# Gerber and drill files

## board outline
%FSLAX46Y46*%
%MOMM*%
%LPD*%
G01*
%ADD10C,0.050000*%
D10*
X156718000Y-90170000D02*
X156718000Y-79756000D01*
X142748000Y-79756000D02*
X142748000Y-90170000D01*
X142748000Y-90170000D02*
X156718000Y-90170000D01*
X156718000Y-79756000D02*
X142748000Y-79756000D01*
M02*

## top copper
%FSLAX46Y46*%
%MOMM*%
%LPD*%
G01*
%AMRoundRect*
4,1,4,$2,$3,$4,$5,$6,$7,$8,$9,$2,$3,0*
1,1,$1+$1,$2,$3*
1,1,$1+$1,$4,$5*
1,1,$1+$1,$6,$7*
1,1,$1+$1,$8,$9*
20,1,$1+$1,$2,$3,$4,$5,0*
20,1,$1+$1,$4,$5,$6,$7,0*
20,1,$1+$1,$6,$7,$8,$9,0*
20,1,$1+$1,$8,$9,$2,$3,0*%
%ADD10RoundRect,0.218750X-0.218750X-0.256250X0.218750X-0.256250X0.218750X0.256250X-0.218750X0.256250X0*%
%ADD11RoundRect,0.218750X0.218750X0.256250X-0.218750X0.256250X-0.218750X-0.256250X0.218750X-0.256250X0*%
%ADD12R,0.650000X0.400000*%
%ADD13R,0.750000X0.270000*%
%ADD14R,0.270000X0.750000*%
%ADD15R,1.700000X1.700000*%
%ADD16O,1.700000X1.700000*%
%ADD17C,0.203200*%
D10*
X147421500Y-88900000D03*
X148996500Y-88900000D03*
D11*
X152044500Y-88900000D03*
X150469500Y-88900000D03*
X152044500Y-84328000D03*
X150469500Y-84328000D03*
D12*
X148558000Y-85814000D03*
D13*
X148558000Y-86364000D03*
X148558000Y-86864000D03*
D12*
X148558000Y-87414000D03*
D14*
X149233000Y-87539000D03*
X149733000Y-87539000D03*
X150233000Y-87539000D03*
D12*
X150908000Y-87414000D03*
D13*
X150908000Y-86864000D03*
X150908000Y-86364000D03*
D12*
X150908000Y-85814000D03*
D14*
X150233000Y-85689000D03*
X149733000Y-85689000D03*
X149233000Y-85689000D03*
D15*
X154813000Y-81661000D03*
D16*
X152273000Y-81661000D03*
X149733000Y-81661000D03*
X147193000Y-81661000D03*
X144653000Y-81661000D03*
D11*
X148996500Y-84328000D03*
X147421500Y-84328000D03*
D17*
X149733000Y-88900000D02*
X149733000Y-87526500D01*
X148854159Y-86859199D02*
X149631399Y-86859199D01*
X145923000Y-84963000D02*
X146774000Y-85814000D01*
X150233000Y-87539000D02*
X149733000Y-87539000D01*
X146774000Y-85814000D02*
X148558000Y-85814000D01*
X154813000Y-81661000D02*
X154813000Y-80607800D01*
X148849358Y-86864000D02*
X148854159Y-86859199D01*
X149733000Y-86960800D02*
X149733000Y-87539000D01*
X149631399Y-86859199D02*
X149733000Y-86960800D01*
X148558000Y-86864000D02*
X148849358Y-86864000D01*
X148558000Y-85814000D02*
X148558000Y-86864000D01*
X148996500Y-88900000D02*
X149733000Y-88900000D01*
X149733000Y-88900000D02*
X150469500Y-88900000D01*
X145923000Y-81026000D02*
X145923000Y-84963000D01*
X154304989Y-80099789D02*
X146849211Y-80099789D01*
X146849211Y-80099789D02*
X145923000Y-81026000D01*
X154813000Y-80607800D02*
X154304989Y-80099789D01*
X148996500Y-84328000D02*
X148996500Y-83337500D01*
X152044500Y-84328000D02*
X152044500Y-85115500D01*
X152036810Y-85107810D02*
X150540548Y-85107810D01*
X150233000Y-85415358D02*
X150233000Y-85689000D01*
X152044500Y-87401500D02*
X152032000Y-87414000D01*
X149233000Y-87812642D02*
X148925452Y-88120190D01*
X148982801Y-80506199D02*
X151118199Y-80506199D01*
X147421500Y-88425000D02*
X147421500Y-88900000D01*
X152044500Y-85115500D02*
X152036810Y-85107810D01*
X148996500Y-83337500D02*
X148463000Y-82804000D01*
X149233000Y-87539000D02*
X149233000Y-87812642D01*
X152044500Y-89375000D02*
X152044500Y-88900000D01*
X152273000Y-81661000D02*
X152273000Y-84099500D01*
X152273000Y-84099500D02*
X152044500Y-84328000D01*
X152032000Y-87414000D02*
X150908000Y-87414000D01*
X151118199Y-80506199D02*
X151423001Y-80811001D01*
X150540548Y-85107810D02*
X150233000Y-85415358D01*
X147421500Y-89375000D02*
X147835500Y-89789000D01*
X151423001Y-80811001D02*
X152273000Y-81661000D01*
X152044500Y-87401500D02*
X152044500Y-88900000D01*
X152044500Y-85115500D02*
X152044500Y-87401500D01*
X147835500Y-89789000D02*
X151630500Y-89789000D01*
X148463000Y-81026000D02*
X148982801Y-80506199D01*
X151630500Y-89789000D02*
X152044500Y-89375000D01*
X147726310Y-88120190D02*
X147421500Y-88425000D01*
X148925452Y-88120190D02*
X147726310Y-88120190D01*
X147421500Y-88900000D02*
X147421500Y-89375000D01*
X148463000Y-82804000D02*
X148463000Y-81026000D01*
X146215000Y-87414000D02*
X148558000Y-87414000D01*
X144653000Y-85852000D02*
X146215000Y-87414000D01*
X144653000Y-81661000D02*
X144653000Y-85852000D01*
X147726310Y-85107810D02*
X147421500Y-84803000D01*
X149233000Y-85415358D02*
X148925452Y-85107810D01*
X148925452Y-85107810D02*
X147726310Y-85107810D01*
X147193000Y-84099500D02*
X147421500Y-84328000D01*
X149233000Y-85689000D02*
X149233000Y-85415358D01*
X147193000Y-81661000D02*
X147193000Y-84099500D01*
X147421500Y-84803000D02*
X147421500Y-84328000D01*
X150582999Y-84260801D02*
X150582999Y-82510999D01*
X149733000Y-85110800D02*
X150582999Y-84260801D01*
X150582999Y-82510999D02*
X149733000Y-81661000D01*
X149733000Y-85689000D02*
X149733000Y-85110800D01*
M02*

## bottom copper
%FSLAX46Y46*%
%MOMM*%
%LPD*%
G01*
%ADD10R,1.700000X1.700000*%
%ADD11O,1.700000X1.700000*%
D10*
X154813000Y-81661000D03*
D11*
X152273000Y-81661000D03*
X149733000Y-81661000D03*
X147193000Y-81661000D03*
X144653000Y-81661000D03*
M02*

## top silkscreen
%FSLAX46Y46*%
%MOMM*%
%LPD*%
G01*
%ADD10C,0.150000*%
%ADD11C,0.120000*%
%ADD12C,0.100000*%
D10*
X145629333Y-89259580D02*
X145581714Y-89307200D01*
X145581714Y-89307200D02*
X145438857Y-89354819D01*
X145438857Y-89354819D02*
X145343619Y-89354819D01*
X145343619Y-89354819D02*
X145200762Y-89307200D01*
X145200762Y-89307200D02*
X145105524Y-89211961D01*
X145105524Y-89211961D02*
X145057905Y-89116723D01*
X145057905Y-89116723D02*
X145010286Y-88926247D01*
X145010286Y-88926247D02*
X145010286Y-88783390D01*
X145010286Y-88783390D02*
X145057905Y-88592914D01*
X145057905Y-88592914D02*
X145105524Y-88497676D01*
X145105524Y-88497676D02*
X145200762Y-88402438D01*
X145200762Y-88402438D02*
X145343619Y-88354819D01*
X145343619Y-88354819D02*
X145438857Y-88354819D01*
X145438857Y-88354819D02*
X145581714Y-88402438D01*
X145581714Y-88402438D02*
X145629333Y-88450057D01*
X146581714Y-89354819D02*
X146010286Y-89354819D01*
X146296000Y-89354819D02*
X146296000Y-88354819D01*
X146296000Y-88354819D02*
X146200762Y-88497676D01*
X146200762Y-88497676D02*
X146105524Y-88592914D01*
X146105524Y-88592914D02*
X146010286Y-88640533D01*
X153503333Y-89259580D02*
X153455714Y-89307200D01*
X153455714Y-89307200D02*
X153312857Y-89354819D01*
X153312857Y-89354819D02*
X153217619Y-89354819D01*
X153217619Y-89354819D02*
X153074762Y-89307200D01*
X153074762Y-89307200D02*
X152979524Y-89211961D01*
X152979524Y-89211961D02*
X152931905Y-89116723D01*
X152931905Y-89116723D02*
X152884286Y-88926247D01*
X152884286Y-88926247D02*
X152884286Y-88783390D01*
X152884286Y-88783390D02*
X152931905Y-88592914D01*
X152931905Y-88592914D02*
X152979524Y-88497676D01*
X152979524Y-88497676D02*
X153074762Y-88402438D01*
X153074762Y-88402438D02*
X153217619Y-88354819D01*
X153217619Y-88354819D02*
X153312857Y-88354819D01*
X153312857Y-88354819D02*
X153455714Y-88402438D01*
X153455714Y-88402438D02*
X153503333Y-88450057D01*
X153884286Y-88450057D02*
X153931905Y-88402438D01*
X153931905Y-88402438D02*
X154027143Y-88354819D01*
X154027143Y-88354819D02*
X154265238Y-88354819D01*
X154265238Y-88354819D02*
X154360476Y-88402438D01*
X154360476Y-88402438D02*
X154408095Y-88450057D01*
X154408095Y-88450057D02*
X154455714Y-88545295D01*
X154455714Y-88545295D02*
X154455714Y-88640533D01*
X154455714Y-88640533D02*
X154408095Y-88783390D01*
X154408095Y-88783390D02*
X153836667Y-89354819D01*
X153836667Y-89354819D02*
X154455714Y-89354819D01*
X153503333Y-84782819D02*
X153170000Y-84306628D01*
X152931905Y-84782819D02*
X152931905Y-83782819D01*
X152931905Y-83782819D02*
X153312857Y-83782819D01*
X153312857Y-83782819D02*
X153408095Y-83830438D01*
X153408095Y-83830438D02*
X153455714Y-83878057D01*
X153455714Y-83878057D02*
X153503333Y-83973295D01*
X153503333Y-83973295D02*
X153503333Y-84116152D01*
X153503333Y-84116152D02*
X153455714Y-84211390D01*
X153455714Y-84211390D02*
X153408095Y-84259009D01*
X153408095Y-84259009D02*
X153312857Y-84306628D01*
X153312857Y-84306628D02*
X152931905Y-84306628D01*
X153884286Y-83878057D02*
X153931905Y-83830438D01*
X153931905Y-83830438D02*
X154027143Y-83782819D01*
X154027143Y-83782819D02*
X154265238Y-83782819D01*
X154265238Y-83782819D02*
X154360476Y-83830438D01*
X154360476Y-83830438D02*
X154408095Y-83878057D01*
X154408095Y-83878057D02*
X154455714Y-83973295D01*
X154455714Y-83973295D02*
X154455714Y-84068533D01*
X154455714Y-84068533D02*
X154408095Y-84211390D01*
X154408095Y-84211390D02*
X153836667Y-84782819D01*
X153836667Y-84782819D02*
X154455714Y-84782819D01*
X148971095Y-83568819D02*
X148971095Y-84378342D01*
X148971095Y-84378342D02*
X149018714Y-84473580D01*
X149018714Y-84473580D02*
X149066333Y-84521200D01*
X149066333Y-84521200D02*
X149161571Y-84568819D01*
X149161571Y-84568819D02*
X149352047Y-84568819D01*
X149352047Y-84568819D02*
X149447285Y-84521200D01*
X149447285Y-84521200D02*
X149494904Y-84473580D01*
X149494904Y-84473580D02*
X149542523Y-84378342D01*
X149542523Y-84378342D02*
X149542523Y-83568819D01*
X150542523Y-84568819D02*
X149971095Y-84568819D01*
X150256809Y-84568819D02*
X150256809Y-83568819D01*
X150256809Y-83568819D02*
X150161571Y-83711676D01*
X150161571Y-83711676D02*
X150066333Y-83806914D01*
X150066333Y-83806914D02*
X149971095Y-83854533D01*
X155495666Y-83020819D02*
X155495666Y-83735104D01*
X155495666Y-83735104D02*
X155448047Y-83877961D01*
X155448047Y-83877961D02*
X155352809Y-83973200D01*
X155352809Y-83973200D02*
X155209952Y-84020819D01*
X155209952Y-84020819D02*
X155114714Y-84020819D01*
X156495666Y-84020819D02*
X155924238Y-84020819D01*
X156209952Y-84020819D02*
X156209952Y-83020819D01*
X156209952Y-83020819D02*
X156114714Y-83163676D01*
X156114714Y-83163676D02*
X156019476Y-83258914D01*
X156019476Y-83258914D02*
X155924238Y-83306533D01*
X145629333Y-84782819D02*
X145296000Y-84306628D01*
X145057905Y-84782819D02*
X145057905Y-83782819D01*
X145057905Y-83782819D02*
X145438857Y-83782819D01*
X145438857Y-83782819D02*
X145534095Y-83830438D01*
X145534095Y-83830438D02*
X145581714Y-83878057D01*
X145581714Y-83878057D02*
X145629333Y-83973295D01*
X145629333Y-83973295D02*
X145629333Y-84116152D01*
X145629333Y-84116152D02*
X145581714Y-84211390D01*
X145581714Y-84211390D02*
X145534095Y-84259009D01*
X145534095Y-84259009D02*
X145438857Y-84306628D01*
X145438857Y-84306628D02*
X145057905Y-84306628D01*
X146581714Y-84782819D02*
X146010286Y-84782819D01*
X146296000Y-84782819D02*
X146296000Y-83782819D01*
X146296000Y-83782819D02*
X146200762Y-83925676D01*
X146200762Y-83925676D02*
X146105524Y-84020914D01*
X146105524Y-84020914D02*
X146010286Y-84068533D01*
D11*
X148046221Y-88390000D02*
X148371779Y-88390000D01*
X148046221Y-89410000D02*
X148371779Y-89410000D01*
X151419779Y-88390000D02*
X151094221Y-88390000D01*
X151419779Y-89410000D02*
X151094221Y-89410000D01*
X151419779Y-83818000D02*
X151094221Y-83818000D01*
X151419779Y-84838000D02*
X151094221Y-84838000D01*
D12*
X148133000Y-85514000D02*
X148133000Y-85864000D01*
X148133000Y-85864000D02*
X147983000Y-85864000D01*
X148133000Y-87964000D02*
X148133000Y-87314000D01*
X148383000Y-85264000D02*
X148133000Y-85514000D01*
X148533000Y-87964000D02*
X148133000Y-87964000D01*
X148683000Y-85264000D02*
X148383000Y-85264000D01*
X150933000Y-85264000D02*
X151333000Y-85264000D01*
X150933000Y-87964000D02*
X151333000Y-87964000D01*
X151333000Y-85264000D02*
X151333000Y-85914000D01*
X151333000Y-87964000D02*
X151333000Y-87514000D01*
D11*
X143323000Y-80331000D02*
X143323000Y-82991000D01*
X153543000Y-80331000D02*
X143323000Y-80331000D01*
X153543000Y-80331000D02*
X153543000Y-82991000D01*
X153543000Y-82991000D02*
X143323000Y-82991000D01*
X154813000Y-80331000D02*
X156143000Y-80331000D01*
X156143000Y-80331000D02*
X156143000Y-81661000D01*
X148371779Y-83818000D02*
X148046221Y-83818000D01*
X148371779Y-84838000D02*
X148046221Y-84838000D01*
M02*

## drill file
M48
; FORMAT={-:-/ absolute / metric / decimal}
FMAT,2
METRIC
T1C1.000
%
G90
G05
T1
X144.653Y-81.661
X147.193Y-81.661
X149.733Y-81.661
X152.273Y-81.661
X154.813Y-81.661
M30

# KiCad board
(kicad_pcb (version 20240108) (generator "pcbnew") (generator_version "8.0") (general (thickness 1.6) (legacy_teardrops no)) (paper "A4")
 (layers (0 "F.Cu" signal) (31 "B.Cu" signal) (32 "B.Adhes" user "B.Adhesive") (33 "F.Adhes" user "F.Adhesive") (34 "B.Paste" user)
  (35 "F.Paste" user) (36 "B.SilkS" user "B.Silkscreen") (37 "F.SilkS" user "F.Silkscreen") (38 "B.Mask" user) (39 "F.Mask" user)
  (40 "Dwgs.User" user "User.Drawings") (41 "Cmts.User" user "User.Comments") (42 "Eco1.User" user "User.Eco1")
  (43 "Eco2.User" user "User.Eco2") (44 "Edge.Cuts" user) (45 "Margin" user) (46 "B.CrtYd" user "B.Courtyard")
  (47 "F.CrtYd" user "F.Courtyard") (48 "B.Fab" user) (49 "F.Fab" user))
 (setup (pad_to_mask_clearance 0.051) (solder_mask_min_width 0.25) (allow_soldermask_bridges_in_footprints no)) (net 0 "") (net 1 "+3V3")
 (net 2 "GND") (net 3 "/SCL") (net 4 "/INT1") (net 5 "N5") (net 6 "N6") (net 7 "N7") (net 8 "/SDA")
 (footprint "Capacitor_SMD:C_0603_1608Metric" (layer "F.Cu") (at 148.209 88.9)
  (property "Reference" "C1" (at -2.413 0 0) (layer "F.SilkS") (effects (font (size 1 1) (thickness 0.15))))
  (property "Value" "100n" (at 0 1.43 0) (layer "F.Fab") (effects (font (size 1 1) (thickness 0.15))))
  (fp_line (start -0.162779 -0.51) (end 0.162779 -0.51) (stroke (width 0.12) (type solid)) (layer "F.SilkS"))
  (fp_line (start -0.162779 0.51) (end 0.162779 0.51) (stroke (width 0.12) (type solid)) (layer "F.SilkS"))
  (pad "1" smd roundrect (at -0.7875 0) (size 0.875 0.95) (layers "F.Cu" "F.Paste" "F.Mask") (roundrect_rratio 0.25) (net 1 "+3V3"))
  (pad "2" smd roundrect (at 0.7875 0) (size 0.875 0.95) (layers "F.Cu" "F.Paste" "F.Mask") (roundrect_rratio 0.25) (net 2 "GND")))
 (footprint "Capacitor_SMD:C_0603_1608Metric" (layer "F.Cu") (at 151.257 88.9 180)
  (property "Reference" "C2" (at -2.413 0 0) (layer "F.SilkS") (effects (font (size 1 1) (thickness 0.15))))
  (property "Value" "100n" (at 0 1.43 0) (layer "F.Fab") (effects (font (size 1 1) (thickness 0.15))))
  (fp_line (start -0.162779 0.51) (end 0.162779 0.51) (stroke (width 0.12) (type solid)) (layer "F.SilkS"))
  (fp_line (start -0.162779 -0.51) (end 0.162779 -0.51) (stroke (width 0.12) (type solid)) (layer "F.SilkS"))
  (pad "1" smd roundrect (at -0.7875 0 180) (size 0.875 0.95) (layers "F.Cu" "F.Paste" "F.Mask") (roundrect_rratio 0.25) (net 1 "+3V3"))
  (pad "2" smd roundrect (at 0.7875 0 180) (size 0.875 0.95) (layers "F.Cu" "F.Paste" "F.Mask") (roundrect_rratio 0.25) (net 2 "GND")))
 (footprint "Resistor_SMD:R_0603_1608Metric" (layer "F.Cu") (at 151.257 84.328 180)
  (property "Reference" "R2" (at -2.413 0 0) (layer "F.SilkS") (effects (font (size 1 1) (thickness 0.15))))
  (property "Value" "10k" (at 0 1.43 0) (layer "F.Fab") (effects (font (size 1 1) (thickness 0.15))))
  (fp_line (start -0.162779 0.51) (end 0.162779 0.51) (stroke (width 0.12) (type solid)) (layer "F.SilkS"))
  (fp_line (start -0.162779 -0.51) (end 0.162779 -0.51) (stroke (width 0.12) (type solid)) (layer "F.SilkS"))
  (pad "1" smd roundrect (at -0.7875 0 180) (size 0.875 0.95) (layers "F.Cu" "F.Paste" "F.Mask") (roundrect_rratio 0.25) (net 1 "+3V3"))
  (pad "2" smd roundrect (at 0.7875 0 180) (size 0.875 0.95) (layers "F.Cu" "F.Paste" "F.Mask") (roundrect_rratio 0.25) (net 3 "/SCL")))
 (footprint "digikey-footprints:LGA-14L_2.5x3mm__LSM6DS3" (layer "F.Cu") (at 149.733 86.614)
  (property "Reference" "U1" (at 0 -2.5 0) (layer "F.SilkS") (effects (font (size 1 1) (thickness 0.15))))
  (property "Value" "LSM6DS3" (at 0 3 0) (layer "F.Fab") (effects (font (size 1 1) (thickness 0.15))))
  (fp_line (start -1.6 -1.1) (end -1.6 -0.75) (stroke (width 0.1) (type solid)) (layer "F.SilkS"))
  (fp_line (start -1.6 -0.75) (end -1.75 -0.75) (stroke (width 0.1) (type solid)) (layer "F.SilkS"))
  (fp_line (start -1.6 1.35) (end -1.6 0.7) (stroke (width 0.1) (type solid)) (layer "F.SilkS"))
  (fp_line (start -1.35 -1.35) (end -1.6 -1.1) (stroke (width 0.1) (type solid)) (layer "F.SilkS"))
  (fp_line (start -1.2 1.35) (end -1.6 1.35) (stroke (width 0.1) (type solid)) (layer "F.SilkS"))
  (fp_line (start -1.05 -1.35) (end -1.35 -1.35) (stroke (width 0.1) (type solid)) (layer "F.SilkS"))
  (fp_line (start 1.2 -1.35) (end 1.6 -1.35) (stroke (width 0.1) (type solid)) (layer "F.SilkS"))
  (fp_line (start 1.2 1.35) (end 1.6 1.35) (stroke (width 0.1) (type solid)) (layer "F.SilkS"))
  (fp_line (start 1.6 -1.35) (end 1.6 -0.7) (stroke (width 0.1) (type solid)) (layer "F.SilkS"))
  (fp_line (start 1.6 1.35) (end 1.6 0.9) (stroke (width 0.1) (type solid)) (layer "F.SilkS"))
  (pad "1" smd rect (at -1.175 -0.8) (size 0.65 0.4) (layers "F.Cu" "F.Paste" "F.Mask") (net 2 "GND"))
  (pad "2" smd rect (at -1.175 -0.25) (size 0.75 0.27) (layers "F.Cu" "F.Paste" "F.Mask") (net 2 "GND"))
  (pad "3" smd rect (at -1.175 0.25) (size 0.75 0.27) (layers "F.Cu" "F.Paste" "F.Mask") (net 2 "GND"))
  (pad "4" smd rect (at -1.175 0.8) (size 0.65 0.4) (layers "F.Cu" "F.Paste" "F.Mask") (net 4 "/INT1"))
  (pad "5" smd rect (at -0.5 0.925) (size 0.27 0.75) (layers "F.Cu" "F.Paste" "F.Mask") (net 1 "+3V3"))
  (pad "6" smd rect (at 0 0.925) (size 0.27 0.75) (layers "F.Cu" "F.Paste" "F.Mask") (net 2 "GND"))
  (pad "7" smd rect (at 0.5 0.925) (size 0.27 0.75) (layers "F.Cu" "F.Paste" "F.Mask") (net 2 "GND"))
  (pad "8" smd rect (at 1.175 0.8) (size 0.65 0.4) (layers "F.Cu" "F.Paste" "F.Mask") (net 1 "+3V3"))
  (pad "9" smd rect (at 1.175 0.25) (size 0.75 0.27) (layers "F.Cu" "F.Paste" "F.Mask") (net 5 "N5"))
  (pad "10" smd rect (at 1.175 -0.25) (size 0.75 0.27) (layers "F.Cu" "F.Paste" "F.Mask") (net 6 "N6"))
  (pad "11" smd rect (at 1.175 -0.8) (size 0.65 0.4) (layers "F.Cu" "F.Paste" "F.Mask") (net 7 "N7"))
  (pad "12" smd rect (at 0.5 -0.925) (size 0.27 0.75) (layers "F.Cu" "F.Paste" "F.Mask") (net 1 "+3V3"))
  (pad "13" smd rect (at 0 -0.925) (size 0.27 0.75) (layers "F.Cu" "F.Paste" "F.Mask") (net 3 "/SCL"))
  (pad "14" smd rect (at -0.5 -0.925) (size 0.27 0.75) (layers "F.Cu" "F.Paste" "F.Mask") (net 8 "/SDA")))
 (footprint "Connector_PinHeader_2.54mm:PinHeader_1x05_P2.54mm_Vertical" (layer "F.Cu") (at 154.813 81.661 -90)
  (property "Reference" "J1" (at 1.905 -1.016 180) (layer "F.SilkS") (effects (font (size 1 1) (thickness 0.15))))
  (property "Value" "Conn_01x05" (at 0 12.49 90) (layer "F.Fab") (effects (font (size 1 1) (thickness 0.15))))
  (fp_line (start -1.33 11.49) (end 1.33 11.49) (stroke (width 0.12) (type solid)) (layer "F.SilkS"))
  (fp_line (start -1.33 1.27) (end -1.33 11.49) (stroke (width 0.12) (type solid)) (layer "F.SilkS"))
  (fp_line (start -1.33 1.27) (end 1.33 1.27) (stroke (width 0.12) (type solid)) (layer "F.SilkS"))
  (fp_line (start 1.33 1.27) (end 1.33 11.49) (stroke (width 0.12) (type solid)) (layer "F.SilkS"))
  (fp_line (start -1.33 0) (end -1.33 -1.33) (stroke (width 0.12) (type solid)) (layer "F.SilkS"))
  (fp_line (start -1.33 -1.33) (end 0 -1.33) (stroke (width 0.12) (type solid)) (layer "F.SilkS"))
  (pad "1" thru_hole rect (at 0 0 270) (size 1.7 1.7) (drill 1) (layers "*.Cu" "*.Mask") (remove_unused_layers no) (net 2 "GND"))
  (pad "2" thru_hole oval (at 0 2.54 270) (size 1.7 1.7) (drill 1) (layers "*.Cu" "*.Mask") (remove_unused_layers no) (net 1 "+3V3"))
  (pad "3" thru_hole oval (at 0 5.08 270) (size 1.7 1.7) (drill 1) (layers "*.Cu" "*.Mask") (remove_unused_layers no) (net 3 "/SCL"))
  (pad "4" thru_hole oval (at 0 7.62 270) (size 1.7 1.7) (drill 1) (layers "*.Cu" "*.Mask") (remove_unused_layers no) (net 8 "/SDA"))
  (pad "5" thru_hole oval (at 0 10.16 270) (size 1.7 1.7) (drill 1) (layers "*.Cu" "*.Mask") (remove_unused_layers no) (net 4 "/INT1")))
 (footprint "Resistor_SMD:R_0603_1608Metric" (layer "F.Cu") (at 148.209 84.328 180)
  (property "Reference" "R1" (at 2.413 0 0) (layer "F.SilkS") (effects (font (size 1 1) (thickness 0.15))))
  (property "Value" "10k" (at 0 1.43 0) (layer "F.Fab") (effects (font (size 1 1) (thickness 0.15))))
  (fp_line (start -0.162779 0.51) (end 0.162779 0.51) (stroke (width 0.12) (type solid)) (layer "F.SilkS"))
  (fp_line (start -0.162779 -0.51) (end 0.162779 -0.51) (stroke (width 0.12) (type solid)) (layer "F.SilkS"))
  (pad "1" smd roundrect (at -0.7875 0 180) (size 0.875 0.95) (layers "F.Cu" "F.Paste" "F.Mask") (roundrect_rratio 0.25) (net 1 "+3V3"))
  (pad "2" smd roundrect (at 0.7875 0 180) (size 0.875 0.95) (layers "F.Cu" "F.Paste" "F.Mask") (roundrect_rratio 0.25) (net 8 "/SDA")))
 (gr_line (start 156.718 90.17) (end 156.718 79.756) (stroke (width 0.05) (type solid)) (layer "Edge.Cuts"))
 (gr_line (start 142.748 79.756) (end 142.748 90.17) (stroke (width 0.05) (type solid)) (layer "Edge.Cuts"))
 (gr_line (start 142.748 90.17) (end 156.718 90.17) (stroke (width 0.05) (type solid)) (layer "Edge.Cuts"))
 (gr_line (start 156.718 79.756) (end 142.748 79.756) (stroke (width 0.05) (type solid)) (layer "Edge.Cuts"))
 (segment (start 149.733 88.9) (end 149.733 87.5265) (width 0.2032) (layer "F.Cu") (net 2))
 (segment (start 148.854159 86.859199) (end 149.631399 86.859199) (width 0.2032) (layer "F.Cu") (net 2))
 (segment (start 145.923 84.963) (end 146.774 85.814) (width 0.2032) (layer "F.Cu") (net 2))
 (segment (start 150.233 87.539) (end 149.733 87.539) (width 0.2032) (layer "F.Cu") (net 2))
 (segment (start 146.774 85.814) (end 148.558 85.814) (width 0.2032) (layer "F.Cu") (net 2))
 (segment (start 154.813 81.661) (end 154.813 80.6078) (width 0.2032) (layer "F.Cu") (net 2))
 (segment (start 148.849358 86.864) (end 148.854159 86.859199) (width 0.2032) (layer "F.Cu") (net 2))
 (segment (start 149.733 86.9608) (end 149.733 87.539) (width 0.2032) (layer "F.Cu") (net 2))
 (segment (start 149.631399 86.859199) (end 149.733 86.9608) (width 0.2032) (layer "F.Cu") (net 2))
 (segment (start 148.558 86.864) (end 148.849358 86.864) (width 0.2032) (layer "F.Cu") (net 2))
 (segment (start 148.558 85.814) (end 148.558 86.864) (width 0.2032) (layer "F.Cu") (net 2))
 (segment (start 148.9965 88.9) (end 149.733 88.9) (width 0.2032) (layer "F.Cu") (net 2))
 (segment (start 149.733 88.9) (end 150.4695 88.9) (width 0.2032) (layer "F.Cu") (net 2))
 (segment (start 145.923 81.026) (end 145.923 84.963) (width 0.2032) (layer "F.Cu") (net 2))
 (segment (start 154.304989 80.099789) (end 146.849211 80.099789) (width 0.2032) (layer "F.Cu") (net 2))
 (segment (start 146.849211 80.099789) (end 145.923 81.026) (width 0.2032) (layer "F.Cu") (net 2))
 (segment (start 154.813 80.6078) (end 154.304989 80.099789) (width 0.2032) (layer "F.Cu") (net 2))
 (segment (start 148.9965 84.328) (end 148.9965 83.3375) (width 0.2032) (layer "F.Cu") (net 1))
 (segment (start 152.0445 84.328) (end 152.0445 85.1155) (width 0.2032) (layer "F.Cu") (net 1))
 (segment (start 152.03681 85.10781) (end 150.540548 85.10781) (width 0.2032) (layer "F.Cu") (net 1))
 (segment (start 150.233 85.415358) (end 150.233 85.689) (width 0.2032) (layer "F.Cu") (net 1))
 (segment (start 152.0445 87.4015) (end 152.032 87.414) (width 0.2032) (layer "F.Cu") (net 1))
 (segment (start 149.233 87.812642) (end 148.925452 88.12019) (width 0.2032) (layer "F.Cu") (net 1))
 (segment (start 148.982801 80.506199) (end 151.118199 80.506199) (width 0.2032) (layer "F.Cu") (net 1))
 (segment (start 147.4215 88.425) (end 147.4215 88.9) (width 0.2032) (layer "F.Cu") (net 1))
 (segment (start 152.0445 85.1155) (end 152.03681 85.10781) (width 0.2032) (layer "F.Cu") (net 1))
 (segment (start 148.9965 83.3375) (end 148.463 82.804) (width 0.2032) (layer "F.Cu") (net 1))
 (segment (start 149.233 87.539) (end 149.233 87.812642) (width 0.2032) (layer "F.Cu") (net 1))
 (segment (start 152.0445 89.375) (end 152.0445 88.9) (width 0.2032) (layer "F.Cu") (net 1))
 (segment (start 152.273 81.661) (end 152.273 84.0995) (width 0.2032) (layer "F.Cu") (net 1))
 (segment (start 152.273 84.0995) (end 152.0445 84.328) (width 0.2032) (layer "F.Cu") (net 1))
 (segment (start 152.032 87.414) (end 150.908 87.414) (width 0.2032) (layer "F.Cu") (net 1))
 (segment (start 151.118199 80.506199) (end 151.423001 80.811001) (width 0.2032) (layer "F.Cu") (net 1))
 (segment (start 150.540548 85.10781) (end 150.233 85.415358) (width 0.2032) (layer "F.Cu") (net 1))
 (segment (start 147.4215 89.375) (end 147.8355 89.789) (width 0.2032) (layer "F.Cu") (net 1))
 (segment (start 151.423001 80.811001) (end 152.273 81.661) (width 0.2032) (layer "F.Cu") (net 1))
 (segment (start 152.0445 87.4015) (end 152.0445 88.9) (width 0.2032) (layer "F.Cu") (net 1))
 (segment (start 152.0445 85.1155) (end 152.0445 87.4015) (width 0.2032) (layer "F.Cu") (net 1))
 (segment (start 147.8355 89.789) (end 151.6305 89.789) (width 0.2032) (layer "F.Cu") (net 1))
 (segment (start 148.463 81.026) (end 148.982801 80.506199) (width 0.2032) (layer "F.Cu") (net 1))
 (segment (start 151.6305 89.789) (end 152.0445 89.375) (width 0.2032) (layer "F.Cu") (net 1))
 (segment (start 147.72631 88.12019) (end 147.4215 88.425) (width 0.2032) (layer "F.Cu") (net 1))
 (segment (start 148.925452 88.12019) (end 147.72631 88.12019) (width 0.2032) (layer "F.Cu") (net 1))
 (segment (start 147.4215 88.9) (end 147.4215 89.375) (width 0.2032) (layer "F.Cu") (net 1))
 (segment (start 148.463 82.804) (end 148.463 81.026) (width 0.2032) (layer "F.Cu") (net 1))
 (segment (start 146.215 87.414) (end 148.558 87.414) (width 0.2032) (layer "F.Cu") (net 4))
 (segment (start 144.653 85.852) (end 146.215 87.414) (width 0.2032) (layer "F.Cu") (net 4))
 (segment (start 144.653 81.661) (end 144.653 85.852) (width 0.2032) (layer "F.Cu") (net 4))
 (segment (start 147.72631 85.10781) (end 147.4215 84.803) (width 0.2032) (layer "F.Cu") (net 8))
 (segment (start 149.233 85.415358) (end 148.925452 85.10781) (width 0.2032) (layer "F.Cu") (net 8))
 (segment (start 148.925452 85.10781) (end 147.72631 85.10781) (width 0.2032) (layer "F.Cu") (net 8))
 (segment (start 147.193 84.0995) (end 147.4215 84.328) (width 0.2032) (layer "F.Cu") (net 8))
 (segment (start 149.233 85.689) (end 149.233 85.415358) (width 0.2032) (layer "F.Cu") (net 8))
 (segment (start 147.193 81.661) (end 147.193 84.0995) (width 0.2032) (layer "F.Cu") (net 8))
 (segment (start 147.4215 84.803) (end 147.4215 84.328) (width 0.2032) (layer "F.Cu") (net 8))
 (segment (start 150.582999 84.260801) (end 150.582999 82.510999) (width 0.2032) (layer "F.Cu") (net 3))
 (segment (start 149.733 85.1108) (end 150.582999 84.260801) (width 0.2032) (layer "F.Cu") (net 3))
 (segment (start 150.582999 82.510999) (end 149.733 81.661) (width 0.2032) (layer "F.Cu") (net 3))
 (segment (start 149.733 85.689) (end 149.733 85.1108) (width 0.2032) (layer "F.Cu") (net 3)))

